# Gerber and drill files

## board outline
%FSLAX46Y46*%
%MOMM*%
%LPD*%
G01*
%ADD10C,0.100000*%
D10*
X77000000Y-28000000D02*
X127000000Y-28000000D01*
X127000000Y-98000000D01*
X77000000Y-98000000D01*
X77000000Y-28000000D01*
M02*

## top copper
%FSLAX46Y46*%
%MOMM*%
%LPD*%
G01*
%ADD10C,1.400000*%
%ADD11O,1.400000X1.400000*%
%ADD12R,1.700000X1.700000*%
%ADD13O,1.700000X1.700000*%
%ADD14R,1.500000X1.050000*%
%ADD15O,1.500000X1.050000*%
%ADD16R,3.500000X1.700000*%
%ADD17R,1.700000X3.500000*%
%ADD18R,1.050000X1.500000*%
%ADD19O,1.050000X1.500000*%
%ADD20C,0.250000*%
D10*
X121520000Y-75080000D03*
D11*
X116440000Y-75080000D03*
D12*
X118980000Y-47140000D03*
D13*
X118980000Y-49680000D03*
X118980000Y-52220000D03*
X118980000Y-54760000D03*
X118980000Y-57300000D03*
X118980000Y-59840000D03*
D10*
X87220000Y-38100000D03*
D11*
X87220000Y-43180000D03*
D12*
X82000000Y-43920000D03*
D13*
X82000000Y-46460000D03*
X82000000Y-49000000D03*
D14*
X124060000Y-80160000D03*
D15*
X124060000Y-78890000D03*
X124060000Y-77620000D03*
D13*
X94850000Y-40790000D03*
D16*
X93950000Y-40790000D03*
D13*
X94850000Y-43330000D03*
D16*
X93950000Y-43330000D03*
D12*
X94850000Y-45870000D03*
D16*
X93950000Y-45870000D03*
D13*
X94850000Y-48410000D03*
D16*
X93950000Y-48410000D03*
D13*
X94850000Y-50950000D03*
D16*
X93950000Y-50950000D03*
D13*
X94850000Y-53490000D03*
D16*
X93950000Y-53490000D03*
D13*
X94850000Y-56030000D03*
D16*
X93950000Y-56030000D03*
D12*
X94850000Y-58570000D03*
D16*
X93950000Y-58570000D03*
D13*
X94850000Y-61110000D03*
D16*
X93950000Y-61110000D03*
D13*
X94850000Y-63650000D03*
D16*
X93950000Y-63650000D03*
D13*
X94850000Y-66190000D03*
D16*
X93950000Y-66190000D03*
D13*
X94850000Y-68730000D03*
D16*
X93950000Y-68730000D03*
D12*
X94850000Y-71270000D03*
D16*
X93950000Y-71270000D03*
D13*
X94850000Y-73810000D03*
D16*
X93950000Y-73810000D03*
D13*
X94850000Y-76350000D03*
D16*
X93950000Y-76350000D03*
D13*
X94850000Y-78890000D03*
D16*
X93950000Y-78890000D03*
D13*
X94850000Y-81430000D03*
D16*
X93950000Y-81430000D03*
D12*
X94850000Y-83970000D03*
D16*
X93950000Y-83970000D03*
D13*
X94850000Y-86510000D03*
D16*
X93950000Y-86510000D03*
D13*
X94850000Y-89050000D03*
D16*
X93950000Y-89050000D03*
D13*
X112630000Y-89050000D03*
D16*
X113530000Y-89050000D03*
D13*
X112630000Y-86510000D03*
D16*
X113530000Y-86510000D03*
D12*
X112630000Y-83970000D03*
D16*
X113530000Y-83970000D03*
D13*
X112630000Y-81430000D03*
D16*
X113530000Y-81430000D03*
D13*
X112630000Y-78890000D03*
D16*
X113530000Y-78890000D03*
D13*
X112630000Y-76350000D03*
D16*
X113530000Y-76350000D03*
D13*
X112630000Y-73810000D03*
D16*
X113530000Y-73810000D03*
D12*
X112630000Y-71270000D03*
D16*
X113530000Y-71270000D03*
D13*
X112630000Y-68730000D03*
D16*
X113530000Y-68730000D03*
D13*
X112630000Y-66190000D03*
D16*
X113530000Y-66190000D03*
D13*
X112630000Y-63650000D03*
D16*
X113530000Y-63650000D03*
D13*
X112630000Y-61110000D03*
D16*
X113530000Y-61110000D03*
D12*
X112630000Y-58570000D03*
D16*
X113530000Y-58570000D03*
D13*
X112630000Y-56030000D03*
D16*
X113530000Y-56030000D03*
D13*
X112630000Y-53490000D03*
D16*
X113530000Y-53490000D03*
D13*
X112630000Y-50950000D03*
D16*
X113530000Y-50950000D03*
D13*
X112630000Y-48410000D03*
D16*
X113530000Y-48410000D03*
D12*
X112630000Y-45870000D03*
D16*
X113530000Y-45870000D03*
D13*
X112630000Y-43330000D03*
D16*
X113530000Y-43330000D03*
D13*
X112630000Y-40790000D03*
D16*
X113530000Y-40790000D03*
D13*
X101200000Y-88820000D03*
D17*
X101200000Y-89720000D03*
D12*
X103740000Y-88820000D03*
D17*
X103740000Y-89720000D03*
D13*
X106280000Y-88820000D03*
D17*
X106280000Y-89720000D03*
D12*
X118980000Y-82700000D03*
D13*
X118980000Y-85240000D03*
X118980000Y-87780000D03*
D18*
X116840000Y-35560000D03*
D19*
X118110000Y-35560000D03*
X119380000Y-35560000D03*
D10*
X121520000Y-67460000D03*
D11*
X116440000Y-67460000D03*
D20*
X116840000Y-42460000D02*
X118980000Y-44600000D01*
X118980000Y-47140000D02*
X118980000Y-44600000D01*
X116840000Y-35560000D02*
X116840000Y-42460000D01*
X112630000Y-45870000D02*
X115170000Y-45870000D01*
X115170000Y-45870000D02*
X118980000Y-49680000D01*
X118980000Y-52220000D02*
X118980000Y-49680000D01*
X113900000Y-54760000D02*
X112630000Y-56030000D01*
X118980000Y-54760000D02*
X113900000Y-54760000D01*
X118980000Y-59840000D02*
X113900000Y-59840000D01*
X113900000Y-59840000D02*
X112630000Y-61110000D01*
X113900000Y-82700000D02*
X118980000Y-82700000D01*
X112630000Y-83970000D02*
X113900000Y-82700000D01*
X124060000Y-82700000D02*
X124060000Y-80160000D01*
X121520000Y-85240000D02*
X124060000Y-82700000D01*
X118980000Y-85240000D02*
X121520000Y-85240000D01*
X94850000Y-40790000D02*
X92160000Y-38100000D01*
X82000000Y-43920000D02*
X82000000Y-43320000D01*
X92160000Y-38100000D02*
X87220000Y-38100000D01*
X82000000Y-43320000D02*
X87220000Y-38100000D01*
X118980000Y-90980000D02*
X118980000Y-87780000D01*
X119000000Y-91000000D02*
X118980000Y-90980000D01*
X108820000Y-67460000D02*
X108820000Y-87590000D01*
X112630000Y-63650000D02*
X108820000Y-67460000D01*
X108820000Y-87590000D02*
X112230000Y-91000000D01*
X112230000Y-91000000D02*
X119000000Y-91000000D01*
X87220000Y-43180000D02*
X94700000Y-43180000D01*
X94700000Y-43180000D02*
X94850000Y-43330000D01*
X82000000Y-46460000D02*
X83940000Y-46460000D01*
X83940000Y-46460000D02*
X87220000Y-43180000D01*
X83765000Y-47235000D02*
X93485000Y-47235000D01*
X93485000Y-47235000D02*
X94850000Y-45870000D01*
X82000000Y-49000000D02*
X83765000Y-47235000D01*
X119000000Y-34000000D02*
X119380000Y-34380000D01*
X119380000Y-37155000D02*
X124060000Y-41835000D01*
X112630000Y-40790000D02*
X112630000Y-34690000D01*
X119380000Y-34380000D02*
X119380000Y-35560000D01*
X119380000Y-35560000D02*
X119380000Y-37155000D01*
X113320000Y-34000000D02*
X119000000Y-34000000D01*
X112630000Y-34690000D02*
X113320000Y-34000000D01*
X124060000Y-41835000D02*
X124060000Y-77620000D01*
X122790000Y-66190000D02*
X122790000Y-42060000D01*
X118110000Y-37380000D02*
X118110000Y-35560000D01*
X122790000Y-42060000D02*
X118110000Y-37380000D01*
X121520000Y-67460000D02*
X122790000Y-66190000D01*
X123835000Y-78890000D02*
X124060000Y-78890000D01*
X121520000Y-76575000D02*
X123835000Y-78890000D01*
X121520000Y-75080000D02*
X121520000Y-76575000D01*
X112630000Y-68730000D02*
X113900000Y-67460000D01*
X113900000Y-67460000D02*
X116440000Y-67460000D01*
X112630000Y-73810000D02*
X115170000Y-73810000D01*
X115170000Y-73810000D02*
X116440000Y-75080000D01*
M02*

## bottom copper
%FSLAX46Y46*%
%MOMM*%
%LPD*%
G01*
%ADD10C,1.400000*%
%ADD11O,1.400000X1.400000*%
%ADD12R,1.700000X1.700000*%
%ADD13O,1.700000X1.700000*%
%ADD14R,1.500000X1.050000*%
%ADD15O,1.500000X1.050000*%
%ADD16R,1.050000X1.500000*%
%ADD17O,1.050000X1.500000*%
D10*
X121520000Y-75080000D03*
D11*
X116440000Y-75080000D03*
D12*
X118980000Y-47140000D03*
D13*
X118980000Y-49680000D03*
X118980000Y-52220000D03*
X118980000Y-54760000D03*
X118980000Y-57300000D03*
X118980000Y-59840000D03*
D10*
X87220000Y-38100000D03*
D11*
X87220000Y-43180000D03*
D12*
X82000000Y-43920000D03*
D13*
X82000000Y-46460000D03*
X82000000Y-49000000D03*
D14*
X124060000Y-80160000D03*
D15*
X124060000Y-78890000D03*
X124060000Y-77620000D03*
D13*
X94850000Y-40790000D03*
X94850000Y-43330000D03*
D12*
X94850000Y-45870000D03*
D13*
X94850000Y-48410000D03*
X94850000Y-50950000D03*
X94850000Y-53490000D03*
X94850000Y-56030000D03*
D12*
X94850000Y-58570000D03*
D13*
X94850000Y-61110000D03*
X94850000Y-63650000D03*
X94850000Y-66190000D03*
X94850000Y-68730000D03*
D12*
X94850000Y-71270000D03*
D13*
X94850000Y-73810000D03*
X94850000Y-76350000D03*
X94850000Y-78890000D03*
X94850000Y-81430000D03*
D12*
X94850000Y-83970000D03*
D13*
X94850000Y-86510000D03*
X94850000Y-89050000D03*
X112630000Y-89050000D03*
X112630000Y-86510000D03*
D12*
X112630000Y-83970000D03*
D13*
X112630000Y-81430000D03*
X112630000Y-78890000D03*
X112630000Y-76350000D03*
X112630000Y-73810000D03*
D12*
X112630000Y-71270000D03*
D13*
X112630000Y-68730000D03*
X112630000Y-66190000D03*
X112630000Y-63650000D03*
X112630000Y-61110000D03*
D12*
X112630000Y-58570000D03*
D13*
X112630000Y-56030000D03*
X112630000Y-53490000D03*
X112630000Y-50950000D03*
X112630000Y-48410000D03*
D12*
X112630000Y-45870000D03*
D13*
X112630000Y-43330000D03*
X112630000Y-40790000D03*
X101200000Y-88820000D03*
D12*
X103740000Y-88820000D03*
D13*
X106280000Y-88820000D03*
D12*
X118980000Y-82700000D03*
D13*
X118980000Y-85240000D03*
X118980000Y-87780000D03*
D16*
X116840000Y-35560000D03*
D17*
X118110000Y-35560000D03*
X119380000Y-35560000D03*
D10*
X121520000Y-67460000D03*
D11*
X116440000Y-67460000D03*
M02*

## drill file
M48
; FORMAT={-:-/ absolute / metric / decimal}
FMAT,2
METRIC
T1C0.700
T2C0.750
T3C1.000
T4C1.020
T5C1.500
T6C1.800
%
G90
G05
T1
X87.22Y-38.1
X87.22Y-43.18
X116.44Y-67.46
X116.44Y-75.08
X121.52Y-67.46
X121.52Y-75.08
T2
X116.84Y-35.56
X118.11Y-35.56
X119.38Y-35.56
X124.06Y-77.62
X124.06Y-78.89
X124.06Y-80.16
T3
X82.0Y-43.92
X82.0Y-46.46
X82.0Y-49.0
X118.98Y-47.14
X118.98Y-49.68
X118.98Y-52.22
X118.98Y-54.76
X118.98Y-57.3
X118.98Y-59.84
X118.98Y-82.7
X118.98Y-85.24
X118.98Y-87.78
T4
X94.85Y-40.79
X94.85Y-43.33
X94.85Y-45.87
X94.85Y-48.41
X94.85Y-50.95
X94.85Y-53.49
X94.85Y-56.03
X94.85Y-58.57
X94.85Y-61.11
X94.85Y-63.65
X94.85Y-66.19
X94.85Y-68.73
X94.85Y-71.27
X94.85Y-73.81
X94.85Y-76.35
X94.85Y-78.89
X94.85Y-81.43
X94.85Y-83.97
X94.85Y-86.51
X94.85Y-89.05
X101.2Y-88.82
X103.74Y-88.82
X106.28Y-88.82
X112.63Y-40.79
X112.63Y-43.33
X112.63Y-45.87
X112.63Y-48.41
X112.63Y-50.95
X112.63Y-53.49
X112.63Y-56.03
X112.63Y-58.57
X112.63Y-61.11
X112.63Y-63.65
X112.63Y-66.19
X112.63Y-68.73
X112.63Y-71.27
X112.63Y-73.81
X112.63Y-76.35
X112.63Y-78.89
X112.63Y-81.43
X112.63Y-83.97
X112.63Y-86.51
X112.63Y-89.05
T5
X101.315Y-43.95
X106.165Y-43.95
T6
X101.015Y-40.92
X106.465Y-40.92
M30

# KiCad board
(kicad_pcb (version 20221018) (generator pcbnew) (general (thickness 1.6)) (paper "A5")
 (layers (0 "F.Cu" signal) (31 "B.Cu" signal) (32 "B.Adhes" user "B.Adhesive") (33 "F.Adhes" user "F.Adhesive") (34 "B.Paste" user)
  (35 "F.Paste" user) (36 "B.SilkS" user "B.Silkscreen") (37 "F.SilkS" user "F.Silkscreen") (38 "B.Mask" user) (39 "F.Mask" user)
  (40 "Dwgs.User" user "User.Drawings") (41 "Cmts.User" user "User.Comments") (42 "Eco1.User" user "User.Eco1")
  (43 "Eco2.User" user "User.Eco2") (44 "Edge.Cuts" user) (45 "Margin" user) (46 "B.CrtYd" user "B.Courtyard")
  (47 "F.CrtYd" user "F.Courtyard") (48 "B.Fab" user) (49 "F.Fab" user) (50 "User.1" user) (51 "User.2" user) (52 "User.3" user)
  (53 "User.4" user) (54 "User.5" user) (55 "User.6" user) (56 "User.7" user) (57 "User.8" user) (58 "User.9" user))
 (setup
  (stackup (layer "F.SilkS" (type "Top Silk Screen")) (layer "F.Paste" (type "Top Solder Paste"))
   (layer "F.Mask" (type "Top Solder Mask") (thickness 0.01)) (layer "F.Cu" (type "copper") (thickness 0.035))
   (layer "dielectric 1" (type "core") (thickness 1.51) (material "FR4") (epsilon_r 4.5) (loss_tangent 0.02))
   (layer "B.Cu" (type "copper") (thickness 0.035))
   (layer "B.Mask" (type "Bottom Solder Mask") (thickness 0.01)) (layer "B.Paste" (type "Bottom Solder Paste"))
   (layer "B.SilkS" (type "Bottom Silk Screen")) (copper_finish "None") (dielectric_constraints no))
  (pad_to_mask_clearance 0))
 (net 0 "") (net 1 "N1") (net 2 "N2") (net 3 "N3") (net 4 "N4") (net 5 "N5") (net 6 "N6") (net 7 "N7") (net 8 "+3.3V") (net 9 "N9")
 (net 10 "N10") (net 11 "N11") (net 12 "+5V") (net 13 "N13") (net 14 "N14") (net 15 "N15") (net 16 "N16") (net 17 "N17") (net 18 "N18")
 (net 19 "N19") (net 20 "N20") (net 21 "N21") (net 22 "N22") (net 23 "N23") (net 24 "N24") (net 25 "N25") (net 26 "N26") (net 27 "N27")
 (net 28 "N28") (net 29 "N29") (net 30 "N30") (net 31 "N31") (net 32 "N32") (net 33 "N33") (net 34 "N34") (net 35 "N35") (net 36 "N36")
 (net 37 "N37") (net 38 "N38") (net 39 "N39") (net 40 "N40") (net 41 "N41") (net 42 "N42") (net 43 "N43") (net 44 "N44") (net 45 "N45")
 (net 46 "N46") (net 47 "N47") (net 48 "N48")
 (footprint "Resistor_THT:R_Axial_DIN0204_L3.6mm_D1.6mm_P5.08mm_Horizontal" (layer "F.Cu") (at 121.52 75.08 180)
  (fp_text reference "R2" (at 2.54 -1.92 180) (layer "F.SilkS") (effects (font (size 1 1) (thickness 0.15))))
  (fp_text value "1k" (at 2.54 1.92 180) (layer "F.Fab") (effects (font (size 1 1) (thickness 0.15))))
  (pad "1" thru_hole circle (at 0 0 180) (size 1.4 1.4) (drill 0.7) (layers "*.Cu" "*.Mask") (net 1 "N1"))
  (pad "2" thru_hole oval (at 5.08 0 180) (size 1.4 1.4) (drill 0.7) (layers "*.Cu" "*.Mask") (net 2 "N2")))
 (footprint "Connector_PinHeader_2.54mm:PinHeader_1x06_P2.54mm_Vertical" (layer "F.Cu") (at 118.98 47.14)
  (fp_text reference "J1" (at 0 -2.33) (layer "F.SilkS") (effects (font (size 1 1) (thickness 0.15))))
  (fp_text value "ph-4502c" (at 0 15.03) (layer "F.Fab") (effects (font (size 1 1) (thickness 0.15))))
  (pad "1" thru_hole rect (at 0 0) (size 1.7 1.7) (drill 1) (layers "*.Cu" "*.Mask") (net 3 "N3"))
  (pad "2" thru_hole oval (at 0 2.54) (size 1.7 1.7) (drill 1) (layers "*.Cu" "*.Mask") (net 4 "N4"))
  (pad "3" thru_hole oval (at 0 5.08) (size 1.7 1.7) (drill 1) (layers "*.Cu" "*.Mask") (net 4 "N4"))
  (pad "4" thru_hole oval (at 0 7.62) (size 1.7 1.7) (drill 1) (layers "*.Cu" "*.Mask") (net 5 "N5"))
  (pad "5" thru_hole oval (at 0 10.16) (size 1.7 1.7) (drill 1) (layers "*.Cu" "*.Mask") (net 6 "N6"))
  (pad "6" thru_hole oval (at 0 12.7) (size 1.7 1.7) (drill 1) (layers "*.Cu" "*.Mask") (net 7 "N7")))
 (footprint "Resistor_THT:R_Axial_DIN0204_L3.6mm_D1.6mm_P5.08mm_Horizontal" (layer "F.Cu") (at 87.22 38.1 -90)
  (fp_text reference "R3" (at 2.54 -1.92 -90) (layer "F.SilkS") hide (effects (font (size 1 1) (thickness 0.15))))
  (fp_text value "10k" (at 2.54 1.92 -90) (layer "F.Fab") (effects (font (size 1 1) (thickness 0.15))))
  (pad "1" thru_hole circle (at 0 0 270) (size 1.4 1.4) (drill 0.7) (layers "*.Cu" "*.Mask") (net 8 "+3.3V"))
  (pad "2" thru_hole oval (at 5.08 0 270) (size 1.4 1.4) (drill 0.7) (layers "*.Cu" "*.Mask") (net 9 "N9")))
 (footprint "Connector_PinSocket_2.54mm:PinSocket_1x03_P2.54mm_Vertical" (layer "F.Cu") (at 82 43.92)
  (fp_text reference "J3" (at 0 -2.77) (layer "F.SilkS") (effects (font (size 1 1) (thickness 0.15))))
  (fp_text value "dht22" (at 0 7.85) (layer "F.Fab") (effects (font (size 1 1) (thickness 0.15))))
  (pad "1" thru_hole rect (at 0 0) (size 1.7 1.7) (drill 1) (layers "*.Cu" "*.Mask") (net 8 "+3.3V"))
  (pad "2" thru_hole oval (at 0 2.54) (size 1.7 1.7) (drill 1) (layers "*.Cu" "*.Mask") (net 9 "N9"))
  (pad "3" thru_hole oval (at 0 5.08) (size 1.7 1.7) (drill 1) (layers "*.Cu" "*.Mask") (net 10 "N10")))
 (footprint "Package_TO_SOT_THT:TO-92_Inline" (layer "F.Cu") (at 124.06 80.16 90)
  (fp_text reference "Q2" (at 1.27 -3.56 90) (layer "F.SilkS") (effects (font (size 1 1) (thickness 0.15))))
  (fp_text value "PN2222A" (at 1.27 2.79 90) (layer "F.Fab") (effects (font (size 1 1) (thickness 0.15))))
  (pad "1" thru_hole rect (at 0 0 90) (size 1.05 1.5) (drill 0.75) (layers "*.Cu" "*.Mask") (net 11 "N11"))
  (pad "2" thru_hole oval (at 1.27 0 90) (size 1.05 1.5) (drill 0.75) (layers "*.Cu" "*.Mask") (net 1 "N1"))
  (pad "3" thru_hole oval (at 2.54 0 90) (size 1.05 1.5) (drill 0.75) (layers "*.Cu" "*.Mask") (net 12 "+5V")))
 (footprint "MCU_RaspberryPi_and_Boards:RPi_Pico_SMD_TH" (layer "F.Cu") (at 103.74 64.92)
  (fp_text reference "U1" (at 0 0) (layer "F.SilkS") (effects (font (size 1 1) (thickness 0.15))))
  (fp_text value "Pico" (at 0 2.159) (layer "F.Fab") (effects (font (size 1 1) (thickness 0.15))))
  (pad "" np_thru_hole oval (at -2.725 -24) (size 1.8 1.8) (drill 1.8) (layers "*.Cu" "*.Mask"))
  (pad "" np_thru_hole oval (at -2.425 -20.97) (size 1.5 1.5) (drill 1.5) (layers "*.Cu" "*.Mask"))
  (pad "" np_thru_hole oval (at 2.425 -20.97) (size 1.5 1.5) (drill 1.5) (layers "*.Cu" "*.Mask"))
  (pad "" np_thru_hole oval (at 2.725 -24) (size 1.8 1.8) (drill 1.8) (layers "*.Cu" "*.Mask"))
  (pad "1" thru_hole oval (at -8.89 -24.13) (size 1.7 1.7) (drill 1.02) (layers "*.Cu" "*.Mask") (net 8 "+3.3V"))
  (pad "1" smd rect (at -8.89 -24.13) (size 3.5 1.7) (drill (offset -0.9 0)) (layers "F.Cu" "F.Mask") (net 8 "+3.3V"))
  (pad "2" thru_hole oval (at -8.89 -21.59) (size 1.7 1.7) (drill 1.02) (layers "*.Cu" "*.Mask") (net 9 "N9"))
  (pad "2" smd rect (at -8.89 -21.59) (size 3.5 1.7) (drill (offset -0.9 0)) (layers "F.Cu" "F.Mask") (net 9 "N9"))
  (pad "3" thru_hole rect (at -8.89 -19.05) (size 1.7 1.7) (drill 1.02) (layers "*.Cu" "*.Mask") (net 10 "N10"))
  (pad "3" smd rect (at -8.89 -19.05) (size 3.5 1.7) (drill (offset -0.9 0)) (layers "F.Cu" "F.Mask") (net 10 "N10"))
  (pad "4" thru_hole oval (at -8.89 -16.51) (size 1.7 1.7) (drill 1.02) (layers "*.Cu" "*.Mask") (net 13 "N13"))
  (pad "4" smd rect (at -8.89 -16.51) (size 3.5 1.7) (drill (offset -0.9 0)) (layers "F.Cu" "F.Mask") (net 13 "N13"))
  (pad "5" thru_hole oval (at -8.89 -13.97) (size 1.7 1.7) (drill 1.02) (layers "*.Cu" "*.Mask") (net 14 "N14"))
  (pad "5" smd rect (at -8.89 -13.97) (size 3.5 1.7) (drill (offset -0.9 0)) (layers "F.Cu" "F.Mask") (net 14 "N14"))
  (pad "6" thru_hole oval (at -8.89 -11.43) (size 1.7 1.7) (drill 1.02) (layers "*.Cu" "*.Mask") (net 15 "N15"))
  (pad "6" smd rect (at -8.89 -11.43) (size 3.5 1.7) (drill (offset -0.9 0)) (layers "F.Cu" "F.Mask") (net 15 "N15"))
  (pad "7" thru_hole oval (at -8.89 -8.89) (size 1.7 1.7) (drill 1.02) (layers "*.Cu" "*.Mask") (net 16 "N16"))
  (pad "7" smd rect (at -8.89 -8.89) (size 3.5 1.7) (drill (offset -0.9 0)) (layers "F.Cu" "F.Mask") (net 16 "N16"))
  (pad "8" thru_hole rect (at -8.89 -6.35) (size 1.7 1.7) (drill 1.02) (layers "*.Cu" "*.Mask") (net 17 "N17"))
  (pad "8" smd rect (at -8.89 -6.35) (size 3.5 1.7) (drill (offset -0.9 0)) (layers "F.Cu" "F.Mask") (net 17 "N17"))
  (pad "9" thru_hole oval (at -8.89 -3.81) (size 1.7 1.7) (drill 1.02) (layers "*.Cu" "*.Mask") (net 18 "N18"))
  (pad "9" smd rect (at -8.89 -3.81) (size 3.5 1.7) (drill (offset -0.9 0)) (layers "F.Cu" "F.Mask") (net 18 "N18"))
  (pad "10" thru_hole oval (at -8.89 -1.27) (size 1.7 1.7) (drill 1.02) (layers "*.Cu" "*.Mask") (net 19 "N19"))
  (pad "10" smd rect (at -8.89 -1.27) (size 3.5 1.7) (drill (offset -0.9 0)) (layers "F.Cu" "F.Mask") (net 19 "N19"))
  (pad "11" thru_hole oval (at -8.89 1.27) (size 1.7 1.7) (drill 1.02) (layers "*.Cu" "*.Mask") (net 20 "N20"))
  (pad "11" smd rect (at -8.89 1.27) (size 3.5 1.7) (drill (offset -0.9 0)) (layers "F.Cu" "F.Mask") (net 20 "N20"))
  (pad "12" thru_hole oval (at -8.89 3.81) (size 1.7 1.7) (drill 1.02) (layers "*.Cu" "*.Mask") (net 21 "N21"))
  (pad "12" smd rect (at -8.89 3.81) (size 3.5 1.7) (drill (offset -0.9 0)) (layers "F.Cu" "F.Mask") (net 21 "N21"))
  (pad "13" thru_hole rect (at -8.89 6.35) (size 1.7 1.7) (drill 1.02) (layers "*.Cu" "*.Mask") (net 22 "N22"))
  (pad "13" smd rect (at -8.89 6.35) (size 3.5 1.7) (drill (offset -0.9 0)) (layers "F.Cu" "F.Mask") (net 22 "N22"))
  (pad "14" thru_hole oval (at -8.89 8.89) (size 1.7 1.7) (drill 1.02) (layers "*.Cu" "*.Mask") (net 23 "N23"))
  (pad "14" smd rect (at -8.89 8.89) (size 3.5 1.7) (drill (offset -0.9 0)) (layers "F.Cu" "F.Mask") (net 23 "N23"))
  (pad "15" thru_hole oval (at -8.89 11.43) (size 1.7 1.7) (drill 1.02) (layers "*.Cu" "*.Mask") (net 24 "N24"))
  (pad "15" smd rect (at -8.89 11.43) (size 3.5 1.7) (drill (offset -0.9 0)) (layers "F.Cu" "F.Mask") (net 24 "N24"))
  (pad "16" thru_hole oval (at -8.89 13.97) (size 1.7 1.7) (drill 1.02) (layers "*.Cu" "*.Mask") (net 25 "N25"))
  (pad "16" smd rect (at -8.89 13.97) (size 3.5 1.7) (drill (offset -0.9 0)) (layers "F.Cu" "F.Mask") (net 25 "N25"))
  (pad "17" thru_hole oval (at -8.89 16.51) (size 1.7 1.7) (drill 1.02) (layers "*.Cu" "*.Mask") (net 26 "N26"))
  (pad "17" smd rect (at -8.89 16.51) (size 3.5 1.7) (drill (offset -0.9 0)) (layers "F.Cu" "F.Mask") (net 26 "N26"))
  (pad "18" thru_hole rect (at -8.89 19.05) (size 1.7 1.7) (drill 1.02) (layers "*.Cu" "*.Mask") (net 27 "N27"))
  (pad "18" smd rect (at -8.89 19.05) (size 3.5 1.7) (drill (offset -0.9 0)) (layers "F.Cu" "F.Mask") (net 27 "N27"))
  (pad "19" thru_hole oval (at -8.89 21.59) (size 1.7 1.7) (drill 1.02) (layers "*.Cu" "*.Mask") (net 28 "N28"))
  (pad "19" smd rect (at -8.89 21.59) (size 3.5 1.7) (drill (offset -0.9 0)) (layers "F.Cu" "F.Mask") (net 28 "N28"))
  (pad "20" thru_hole oval (at -8.89 24.13) (size 1.7 1.7) (drill 1.02) (layers "*.Cu" "*.Mask") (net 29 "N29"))
  (pad "20" smd rect (at -8.89 24.13) (size 3.5 1.7) (drill (offset -0.9 0)) (layers "F.Cu" "F.Mask") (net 29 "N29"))
  (pad "21" thru_hole oval (at 8.89 24.13) (size 1.7 1.7) (drill 1.02) (layers "*.Cu" "*.Mask") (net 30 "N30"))
  (pad "21" smd rect (at 8.89 24.13) (size 3.5 1.7) (drill (offset 0.9 0)) (layers "F.Cu" "F.Mask") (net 30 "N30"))
  (pad "22" thru_hole oval (at 8.89 21.59) (size 1.7 1.7) (drill 1.02) (layers "*.Cu" "*.Mask") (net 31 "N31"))
  (pad "22" smd rect (at 8.89 21.59) (size 3.5 1.7) (drill (offset 0.9 0)) (layers "F.Cu" "F.Mask") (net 31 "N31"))
  (pad "23" thru_hole rect (at 8.89 19.05) (size 1.7 1.7) (drill 1.02) (layers "*.Cu" "*.Mask") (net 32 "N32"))
  (pad "23" smd rect (at 8.89 19.05) (size 3.5 1.7) (drill (offset 0.9 0)) (layers "F.Cu" "F.Mask") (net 32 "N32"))
  (pad "24" thru_hole oval (at 8.89 16.51) (size 1.7 1.7) (drill 1.02) (layers "*.Cu" "*.Mask") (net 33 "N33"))
  (pad "24" smd rect (at 8.89 16.51) (size 3.5 1.7) (drill (offset 0.9 0)) (layers "F.Cu" "F.Mask") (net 33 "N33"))
  (pad "25" thru_hole oval (at 8.89 13.97) (size 1.7 1.7) (drill 1.02) (layers "*.Cu" "*.Mask") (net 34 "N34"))
  (pad "25" smd rect (at 8.89 13.97) (size 3.5 1.7) (drill (offset 0.9 0)) (layers "F.Cu" "F.Mask") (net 34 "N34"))
  (pad "26" thru_hole oval (at 8.89 11.43) (size 1.7 1.7) (drill 1.02) (layers "*.Cu" "*.Mask") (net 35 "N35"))
  (pad "26" smd rect (at 8.89 11.43) (size 3.5 1.7) (drill (offset 0.9 0)) (layers "F.Cu" "F.Mask") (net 35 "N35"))
  (pad "27" thru_hole oval (at 8.89 8.89) (size 1.7 1.7) (drill 1.02) (layers "*.Cu" "*.Mask") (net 2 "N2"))
  (pad "27" smd rect (at 8.89 8.89) (size 3.5 1.7) (drill (offset 0.9 0)) (layers "F.Cu" "F.Mask") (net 2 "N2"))
  (pad "28" thru_hole rect (at 8.89 6.35) (size 1.7 1.7) (drill 1.02) (layers "*.Cu" "*.Mask") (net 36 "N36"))
  (pad "28" smd rect (at 8.89 6.35) (size 3.5 1.7) (drill (offset 0.9 0)) (layers "F.Cu" "F.Mask") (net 36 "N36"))
  (pad "29" thru_hole oval (at 8.89 3.81) (size 1.7 1.7) (drill 1.02) (layers "*.Cu" "*.Mask") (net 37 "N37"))
  (pad "29" smd rect (at 8.89 3.81) (size 3.5 1.7) (drill (offset 0.9 0)) (layers "F.Cu" "F.Mask") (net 37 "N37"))
  (pad "30" thru_hole oval (at 8.89 1.27) (size 1.7 1.7) (drill 1.02) (layers "*.Cu" "*.Mask") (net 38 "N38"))
  (pad "30" smd rect (at 8.89 1.27) (size 3.5 1.7) (drill (offset 0.9 0)) (layers "F.Cu" "F.Mask") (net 38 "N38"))
  (pad "31" thru_hole oval (at 8.89 -1.27) (size 1.7 1.7) (drill 1.02) (layers "*.Cu" "*.Mask") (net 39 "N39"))
  (pad "31" smd rect (at 8.89 -1.27) (size 3.5 1.7) (drill (offset 0.9 0)) (layers "F.Cu" "F.Mask") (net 39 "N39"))
  (pad "32" thru_hole oval (at 8.89 -3.81) (size 1.7 1.7) (drill 1.02) (layers "*.Cu" "*.Mask") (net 7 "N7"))
  (pad "32" smd rect (at 8.89 -3.81) (size 3.5 1.7) (drill (offset 0.9 0)) (layers "F.Cu" "F.Mask") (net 7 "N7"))
  (pad "33" thru_hole rect (at 8.89 -6.35) (size 1.7 1.7) (drill 1.02) (layers "*.Cu" "*.Mask") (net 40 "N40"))
  (pad "33" smd rect (at 8.89 -6.35) (size 3.5 1.7) (drill (offset 0.9 0)) (layers "F.Cu" "F.Mask") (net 40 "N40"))
  (pad "34" thru_hole oval (at 8.89 -8.89) (size 1.7 1.7) (drill 1.02) (layers "*.Cu" "*.Mask") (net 5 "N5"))
  (pad "34" smd rect (at 8.89 -8.89) (size 3.5 1.7) (drill (offset 0.9 0)) (layers "F.Cu" "F.Mask") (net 5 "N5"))
  (pad "35" thru_hole oval (at 8.89 -11.43) (size 1.7 1.7) (drill 1.02) (layers "*.Cu" "*.Mask") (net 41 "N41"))
  (pad "35" smd rect (at 8.89 -11.43) (size 3.5 1.7) (drill (offset 0.9 0)) (layers "F.Cu" "F.Mask") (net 41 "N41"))
  (pad "36" thru_hole oval (at 8.89 -13.97) (size 1.7 1.7) (drill 1.02) (layers "*.Cu" "*.Mask") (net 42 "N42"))
  (pad "36" smd rect (at 8.89 -13.97) (size 3.5 1.7) (drill (offset 0.9 0)) (layers "F.Cu" "F.Mask") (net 42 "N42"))
  (pad "37" thru_hole oval (at 8.89 -16.51) (size 1.7 1.7) (drill 1.02) (layers "*.Cu" "*.Mask") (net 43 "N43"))
  (pad "37" smd rect (at 8.89 -16.51) (size 3.5 1.7) (drill (offset 0.9 0)) (layers "F.Cu" "F.Mask") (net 43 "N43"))
  (pad "38" thru_hole rect (at 8.89 -19.05) (size 1.7 1.7) (drill 1.02) (layers "*.Cu" "*.Mask") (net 4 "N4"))
  (pad "38" smd rect (at 8.89 -19.05) (size 3.5 1.7) (drill (offset 0.9 0)) (layers "F.Cu" "F.Mask") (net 4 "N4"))
  (pad "39" thru_hole oval (at 8.89 -21.59) (size 1.7 1.7) (drill 1.02) (layers "*.Cu" "*.Mask") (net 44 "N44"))
  (pad "39" smd rect (at 8.89 -21.59) (size 3.5 1.7) (drill (offset 0.9 0)) (layers "F.Cu" "F.Mask") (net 44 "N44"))
  (pad "40" thru_hole oval (at 8.89 -24.13) (size 1.7 1.7) (drill 1.02) (layers "*.Cu" "*.Mask") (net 12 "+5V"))
  (pad "40" smd rect (at 8.89 -24.13) (size 3.5 1.7) (drill (offset 0.9 0)) (layers "F.Cu" "F.Mask") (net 12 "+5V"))
  (pad "41" thru_hole oval (at -2.54 23.9) (size 1.7 1.7) (drill 1.02) (layers "*.Cu" "*.Mask") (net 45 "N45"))
  (pad "41" smd rect (at -2.54 23.9 90) (size 3.5 1.7) (drill (offset -0.9 0)) (layers "F.Cu" "F.Mask") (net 45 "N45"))
  (pad "42" thru_hole rect (at 0 23.9) (size 1.7 1.7) (drill 1.02) (layers "*.Cu" "*.Mask") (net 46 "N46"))
  (pad "42" smd rect (at 0 23.9 90) (size 3.5 1.7) (drill (offset -0.9 0)) (layers "F.Cu" "F.Mask") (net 46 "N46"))
  (pad "43" thru_hole oval (at 2.54 23.9) (size 1.7 1.7) (drill 1.02) (layers "*.Cu" "*.Mask") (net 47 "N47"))
  (pad "43" smd rect (at 2.54 23.9 90) (size 3.5 1.7) (drill (offset -0.9 0)) (layers "F.Cu" "F.Mask") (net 47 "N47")))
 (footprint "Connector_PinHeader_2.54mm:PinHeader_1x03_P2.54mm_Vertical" (layer "F.Cu") (at 118.98 82.7)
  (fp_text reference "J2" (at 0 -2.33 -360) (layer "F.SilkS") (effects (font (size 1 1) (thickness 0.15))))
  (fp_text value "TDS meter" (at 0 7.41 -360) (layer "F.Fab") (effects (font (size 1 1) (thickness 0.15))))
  (pad "1" thru_hole rect (at 0 0) (size 1.7 1.7) (drill 1) (layers "*.Cu" "*.Mask") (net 32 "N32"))
  (pad "2" thru_hole oval (at 0 2.54) (size 1.7 1.7) (drill 1) (layers "*.Cu" "*.Mask") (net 11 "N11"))
  (pad "3" thru_hole oval (at 0 5.08) (size 1.7 1.7) (drill 1) (layers "*.Cu" "*.Mask") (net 39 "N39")))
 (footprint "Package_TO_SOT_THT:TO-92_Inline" (layer "F.Cu") (at 116.84 35.56)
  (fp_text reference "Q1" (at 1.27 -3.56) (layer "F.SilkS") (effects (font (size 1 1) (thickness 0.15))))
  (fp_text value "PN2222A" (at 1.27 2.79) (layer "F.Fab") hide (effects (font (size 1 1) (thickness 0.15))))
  (pad "1" thru_hole rect (at 0 0) (size 1.05 1.5) (drill 0.75) (layers "*.Cu" "*.Mask") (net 3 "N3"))
  (pad "2" thru_hole oval (at 1.27 0) (size 1.05 1.5) (drill 0.75) (layers "*.Cu" "*.Mask") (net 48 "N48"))
  (pad "3" thru_hole oval (at 2.54 0) (size 1.05 1.5) (drill 0.75) (layers "*.Cu" "*.Mask") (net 12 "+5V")))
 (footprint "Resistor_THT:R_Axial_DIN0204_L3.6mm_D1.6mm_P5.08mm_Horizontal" (layer "F.Cu") (at 121.52 67.46 180)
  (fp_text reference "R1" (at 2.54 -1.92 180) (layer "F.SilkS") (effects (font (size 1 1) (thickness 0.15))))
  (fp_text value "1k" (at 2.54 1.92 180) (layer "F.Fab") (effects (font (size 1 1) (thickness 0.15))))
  (pad "1" thru_hole circle (at 0 0 180) (size 1.4 1.4) (drill 0.7) (layers "*.Cu" "*.Mask") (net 48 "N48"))
  (pad "2" thru_hole oval (at 5.08 0 180) (size 1.4 1.4) (drill 0.7) (layers "*.Cu" "*.Mask") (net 37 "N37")))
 (gr_rect (start 77 28) (end 127 98) (stroke (width 0.1) (type default)) (fill none) (layer "Edge.Cuts"))
 (segment (start 116.84 42.46) (end 118.98 44.6) (width 0.25) (layer "F.Cu") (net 3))
 (segment (start 118.98 47.14) (end 118.98 44.6) (width 0.25) (layer "F.Cu") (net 3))
 (segment (start 116.84 35.56) (end 116.84 42.46) (width 0.25) (layer "F.Cu") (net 3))
 (segment (start 112.63 45.87) (end 115.17 45.87) (width 0.25) (layer "F.Cu") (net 4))
 (segment (start 115.17 45.87) (end 118.98 49.68) (width 0.25) (layer "F.Cu") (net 4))
 (segment (start 118.98 52.22) (end 118.98 49.68) (width 0.25) (layer "F.Cu") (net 4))
 (segment (start 113.9 54.76) (end 112.63 56.03) (width 0.25) (layer "F.Cu") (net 5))
 (segment (start 118.98 54.76) (end 113.9 54.76) (width 0.25) (layer "F.Cu") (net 5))
 (segment (start 118.98 59.84) (end 113.9 59.84) (width 0.25) (layer "F.Cu") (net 7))
 (segment (start 113.9 59.84) (end 112.63 61.11) (width 0.25) (layer "F.Cu") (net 7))
 (segment (start 113.9 82.7) (end 118.98 82.7) (width 0.25) (layer "F.Cu") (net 32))
 (segment (start 112.63 83.97) (end 113.9 82.7) (width 0.25) (layer "F.Cu") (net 32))
 (segment (start 124.06 82.7) (end 124.06 80.16) (width 0.25) (layer "F.Cu") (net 11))
 (segment (start 121.52 85.24) (end 124.06 82.7) (width 0.25) (layer "F.Cu") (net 11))
 (segment (start 118.98 85.24) (end 121.52 85.24) (width 0.25) (layer "F.Cu") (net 11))
 (segment (start 94.85 40.79) (end 92.16 38.1) (width 0.25) (layer "F.Cu") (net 8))
 (segment (start 82 43.92) (end 82 43.32) (width 0.25) (layer "F.Cu") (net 8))
 (segment (start 92.16 38.1) (end 87.22 38.1) (width 0.25) (layer "F.Cu") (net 8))
 (segment (start 82 43.32) (end 87.22 38.1) (width 0.25) (layer "F.Cu") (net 8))
 (segment (start 118.98 90.98) (end 118.98 87.78) (width 0.25) (layer "F.Cu") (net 39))
 (segment (start 119 91) (end 118.98 90.98) (width 0.25) (layer "F.Cu") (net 39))
 (segment (start 108.82 67.46) (end 108.82 87.59) (width 0.25) (layer "F.Cu") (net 39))
 (segment (start 112.63 63.65) (end 108.82 67.46) (width 0.25) (layer "F.Cu") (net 39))
 (segment (start 108.82 87.59) (end 112.23 91) (width 0.25) (layer "F.Cu") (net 39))
 (segment (start 112.23 91) (end 119 91) (width 0.25) (layer "F.Cu") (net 39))
 (segment (start 87.22 43.18) (end 94.7 43.18) (width 0.25) (layer "F.Cu") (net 9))
 (segment (start 94.7 43.18) (end 94.85 43.33) (width 0.25) (layer "F.Cu") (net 9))
 (segment (start 82 46.46) (end 83.94 46.46) (width 0.25) (layer "F.Cu") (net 9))
 (segment (start 83.94 46.46) (end 87.22 43.18) (width 0.25) (layer "F.Cu") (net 9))
 (segment (start 83.765 47.235) (end 93.485 47.235) (width 0.25) (layer "F.Cu") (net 10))
 (segment (start 93.485 47.235) (end 94.85 45.87) (width 0.25) (layer "F.Cu") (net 10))
 (segment (start 82 49) (end 83.765 47.235) (width 0.25) (layer "F.Cu") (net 10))
 (segment (start 119 34) (end 119.38 34.38) (width 0.25) (layer "F.Cu") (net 12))
 (segment (start 119.38 37.155) (end 124.06 41.835) (width 0.25) (layer "F.Cu") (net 12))
 (segment (start 112.63 40.79) (end 112.63 34.69) (width 0.25) (layer "F.Cu") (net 12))
 (segment (start 119.38 34.38) (end 119.38 35.56) (width 0.25) (layer "F.Cu") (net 12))
 (segment (start 119.38 35.56) (end 119.38 37.155) (width 0.25) (layer "F.Cu") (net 12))
 (segment (start 113.32 34) (end 119 34) (width 0.25) (layer "F.Cu") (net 12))
 (segment (start 112.63 34.69) (end 113.32 34) (width 0.25) (layer "F.Cu") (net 12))
 (segment (start 124.06 41.835) (end 124.06 77.62) (width 0.25) (layer "F.Cu") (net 12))
 (segment (start 122.79 66.19) (end 122.79 42.06) (width 0.25) (layer "F.Cu") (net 48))
 (segment (start 118.11 37.38) (end 118.11 35.56) (width 0.25) (layer "F.Cu") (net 48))
 (segment (start 122.79 42.06) (end 118.11 37.38) (width 0.25) (layer "F.Cu") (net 48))
 (segment (start 121.52 67.46) (end 122.79 66.19) (width 0.25) (layer "F.Cu") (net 48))
 (segment (start 123.835 78.89) (end 124.06 78.89) (width 0.25) (layer "F.Cu") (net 1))
 (segment (start 121.52 76.575) (end 123.835 78.89) (width 0.25) (layer "F.Cu") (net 1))
 (segment (start 121.52 75.08) (end 121.52 76.575) (width 0.25) (layer "F.Cu") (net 1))
 (segment (start 112.63 68.73) (end 113.9 67.46) (width 0.25) (layer "F.Cu") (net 37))
 (segment (start 113.9 67.46) (end 116.44 67.46) (width 0.25) (layer "F.Cu") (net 37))
 (segment (start 112.63 73.81) (end 115.17 73.81) (width 0.25) (layer "F.Cu") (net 2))
 (segment (start 115.17 73.81) (end 116.44 75.08) (width 0.25) (layer "F.Cu") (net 2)))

